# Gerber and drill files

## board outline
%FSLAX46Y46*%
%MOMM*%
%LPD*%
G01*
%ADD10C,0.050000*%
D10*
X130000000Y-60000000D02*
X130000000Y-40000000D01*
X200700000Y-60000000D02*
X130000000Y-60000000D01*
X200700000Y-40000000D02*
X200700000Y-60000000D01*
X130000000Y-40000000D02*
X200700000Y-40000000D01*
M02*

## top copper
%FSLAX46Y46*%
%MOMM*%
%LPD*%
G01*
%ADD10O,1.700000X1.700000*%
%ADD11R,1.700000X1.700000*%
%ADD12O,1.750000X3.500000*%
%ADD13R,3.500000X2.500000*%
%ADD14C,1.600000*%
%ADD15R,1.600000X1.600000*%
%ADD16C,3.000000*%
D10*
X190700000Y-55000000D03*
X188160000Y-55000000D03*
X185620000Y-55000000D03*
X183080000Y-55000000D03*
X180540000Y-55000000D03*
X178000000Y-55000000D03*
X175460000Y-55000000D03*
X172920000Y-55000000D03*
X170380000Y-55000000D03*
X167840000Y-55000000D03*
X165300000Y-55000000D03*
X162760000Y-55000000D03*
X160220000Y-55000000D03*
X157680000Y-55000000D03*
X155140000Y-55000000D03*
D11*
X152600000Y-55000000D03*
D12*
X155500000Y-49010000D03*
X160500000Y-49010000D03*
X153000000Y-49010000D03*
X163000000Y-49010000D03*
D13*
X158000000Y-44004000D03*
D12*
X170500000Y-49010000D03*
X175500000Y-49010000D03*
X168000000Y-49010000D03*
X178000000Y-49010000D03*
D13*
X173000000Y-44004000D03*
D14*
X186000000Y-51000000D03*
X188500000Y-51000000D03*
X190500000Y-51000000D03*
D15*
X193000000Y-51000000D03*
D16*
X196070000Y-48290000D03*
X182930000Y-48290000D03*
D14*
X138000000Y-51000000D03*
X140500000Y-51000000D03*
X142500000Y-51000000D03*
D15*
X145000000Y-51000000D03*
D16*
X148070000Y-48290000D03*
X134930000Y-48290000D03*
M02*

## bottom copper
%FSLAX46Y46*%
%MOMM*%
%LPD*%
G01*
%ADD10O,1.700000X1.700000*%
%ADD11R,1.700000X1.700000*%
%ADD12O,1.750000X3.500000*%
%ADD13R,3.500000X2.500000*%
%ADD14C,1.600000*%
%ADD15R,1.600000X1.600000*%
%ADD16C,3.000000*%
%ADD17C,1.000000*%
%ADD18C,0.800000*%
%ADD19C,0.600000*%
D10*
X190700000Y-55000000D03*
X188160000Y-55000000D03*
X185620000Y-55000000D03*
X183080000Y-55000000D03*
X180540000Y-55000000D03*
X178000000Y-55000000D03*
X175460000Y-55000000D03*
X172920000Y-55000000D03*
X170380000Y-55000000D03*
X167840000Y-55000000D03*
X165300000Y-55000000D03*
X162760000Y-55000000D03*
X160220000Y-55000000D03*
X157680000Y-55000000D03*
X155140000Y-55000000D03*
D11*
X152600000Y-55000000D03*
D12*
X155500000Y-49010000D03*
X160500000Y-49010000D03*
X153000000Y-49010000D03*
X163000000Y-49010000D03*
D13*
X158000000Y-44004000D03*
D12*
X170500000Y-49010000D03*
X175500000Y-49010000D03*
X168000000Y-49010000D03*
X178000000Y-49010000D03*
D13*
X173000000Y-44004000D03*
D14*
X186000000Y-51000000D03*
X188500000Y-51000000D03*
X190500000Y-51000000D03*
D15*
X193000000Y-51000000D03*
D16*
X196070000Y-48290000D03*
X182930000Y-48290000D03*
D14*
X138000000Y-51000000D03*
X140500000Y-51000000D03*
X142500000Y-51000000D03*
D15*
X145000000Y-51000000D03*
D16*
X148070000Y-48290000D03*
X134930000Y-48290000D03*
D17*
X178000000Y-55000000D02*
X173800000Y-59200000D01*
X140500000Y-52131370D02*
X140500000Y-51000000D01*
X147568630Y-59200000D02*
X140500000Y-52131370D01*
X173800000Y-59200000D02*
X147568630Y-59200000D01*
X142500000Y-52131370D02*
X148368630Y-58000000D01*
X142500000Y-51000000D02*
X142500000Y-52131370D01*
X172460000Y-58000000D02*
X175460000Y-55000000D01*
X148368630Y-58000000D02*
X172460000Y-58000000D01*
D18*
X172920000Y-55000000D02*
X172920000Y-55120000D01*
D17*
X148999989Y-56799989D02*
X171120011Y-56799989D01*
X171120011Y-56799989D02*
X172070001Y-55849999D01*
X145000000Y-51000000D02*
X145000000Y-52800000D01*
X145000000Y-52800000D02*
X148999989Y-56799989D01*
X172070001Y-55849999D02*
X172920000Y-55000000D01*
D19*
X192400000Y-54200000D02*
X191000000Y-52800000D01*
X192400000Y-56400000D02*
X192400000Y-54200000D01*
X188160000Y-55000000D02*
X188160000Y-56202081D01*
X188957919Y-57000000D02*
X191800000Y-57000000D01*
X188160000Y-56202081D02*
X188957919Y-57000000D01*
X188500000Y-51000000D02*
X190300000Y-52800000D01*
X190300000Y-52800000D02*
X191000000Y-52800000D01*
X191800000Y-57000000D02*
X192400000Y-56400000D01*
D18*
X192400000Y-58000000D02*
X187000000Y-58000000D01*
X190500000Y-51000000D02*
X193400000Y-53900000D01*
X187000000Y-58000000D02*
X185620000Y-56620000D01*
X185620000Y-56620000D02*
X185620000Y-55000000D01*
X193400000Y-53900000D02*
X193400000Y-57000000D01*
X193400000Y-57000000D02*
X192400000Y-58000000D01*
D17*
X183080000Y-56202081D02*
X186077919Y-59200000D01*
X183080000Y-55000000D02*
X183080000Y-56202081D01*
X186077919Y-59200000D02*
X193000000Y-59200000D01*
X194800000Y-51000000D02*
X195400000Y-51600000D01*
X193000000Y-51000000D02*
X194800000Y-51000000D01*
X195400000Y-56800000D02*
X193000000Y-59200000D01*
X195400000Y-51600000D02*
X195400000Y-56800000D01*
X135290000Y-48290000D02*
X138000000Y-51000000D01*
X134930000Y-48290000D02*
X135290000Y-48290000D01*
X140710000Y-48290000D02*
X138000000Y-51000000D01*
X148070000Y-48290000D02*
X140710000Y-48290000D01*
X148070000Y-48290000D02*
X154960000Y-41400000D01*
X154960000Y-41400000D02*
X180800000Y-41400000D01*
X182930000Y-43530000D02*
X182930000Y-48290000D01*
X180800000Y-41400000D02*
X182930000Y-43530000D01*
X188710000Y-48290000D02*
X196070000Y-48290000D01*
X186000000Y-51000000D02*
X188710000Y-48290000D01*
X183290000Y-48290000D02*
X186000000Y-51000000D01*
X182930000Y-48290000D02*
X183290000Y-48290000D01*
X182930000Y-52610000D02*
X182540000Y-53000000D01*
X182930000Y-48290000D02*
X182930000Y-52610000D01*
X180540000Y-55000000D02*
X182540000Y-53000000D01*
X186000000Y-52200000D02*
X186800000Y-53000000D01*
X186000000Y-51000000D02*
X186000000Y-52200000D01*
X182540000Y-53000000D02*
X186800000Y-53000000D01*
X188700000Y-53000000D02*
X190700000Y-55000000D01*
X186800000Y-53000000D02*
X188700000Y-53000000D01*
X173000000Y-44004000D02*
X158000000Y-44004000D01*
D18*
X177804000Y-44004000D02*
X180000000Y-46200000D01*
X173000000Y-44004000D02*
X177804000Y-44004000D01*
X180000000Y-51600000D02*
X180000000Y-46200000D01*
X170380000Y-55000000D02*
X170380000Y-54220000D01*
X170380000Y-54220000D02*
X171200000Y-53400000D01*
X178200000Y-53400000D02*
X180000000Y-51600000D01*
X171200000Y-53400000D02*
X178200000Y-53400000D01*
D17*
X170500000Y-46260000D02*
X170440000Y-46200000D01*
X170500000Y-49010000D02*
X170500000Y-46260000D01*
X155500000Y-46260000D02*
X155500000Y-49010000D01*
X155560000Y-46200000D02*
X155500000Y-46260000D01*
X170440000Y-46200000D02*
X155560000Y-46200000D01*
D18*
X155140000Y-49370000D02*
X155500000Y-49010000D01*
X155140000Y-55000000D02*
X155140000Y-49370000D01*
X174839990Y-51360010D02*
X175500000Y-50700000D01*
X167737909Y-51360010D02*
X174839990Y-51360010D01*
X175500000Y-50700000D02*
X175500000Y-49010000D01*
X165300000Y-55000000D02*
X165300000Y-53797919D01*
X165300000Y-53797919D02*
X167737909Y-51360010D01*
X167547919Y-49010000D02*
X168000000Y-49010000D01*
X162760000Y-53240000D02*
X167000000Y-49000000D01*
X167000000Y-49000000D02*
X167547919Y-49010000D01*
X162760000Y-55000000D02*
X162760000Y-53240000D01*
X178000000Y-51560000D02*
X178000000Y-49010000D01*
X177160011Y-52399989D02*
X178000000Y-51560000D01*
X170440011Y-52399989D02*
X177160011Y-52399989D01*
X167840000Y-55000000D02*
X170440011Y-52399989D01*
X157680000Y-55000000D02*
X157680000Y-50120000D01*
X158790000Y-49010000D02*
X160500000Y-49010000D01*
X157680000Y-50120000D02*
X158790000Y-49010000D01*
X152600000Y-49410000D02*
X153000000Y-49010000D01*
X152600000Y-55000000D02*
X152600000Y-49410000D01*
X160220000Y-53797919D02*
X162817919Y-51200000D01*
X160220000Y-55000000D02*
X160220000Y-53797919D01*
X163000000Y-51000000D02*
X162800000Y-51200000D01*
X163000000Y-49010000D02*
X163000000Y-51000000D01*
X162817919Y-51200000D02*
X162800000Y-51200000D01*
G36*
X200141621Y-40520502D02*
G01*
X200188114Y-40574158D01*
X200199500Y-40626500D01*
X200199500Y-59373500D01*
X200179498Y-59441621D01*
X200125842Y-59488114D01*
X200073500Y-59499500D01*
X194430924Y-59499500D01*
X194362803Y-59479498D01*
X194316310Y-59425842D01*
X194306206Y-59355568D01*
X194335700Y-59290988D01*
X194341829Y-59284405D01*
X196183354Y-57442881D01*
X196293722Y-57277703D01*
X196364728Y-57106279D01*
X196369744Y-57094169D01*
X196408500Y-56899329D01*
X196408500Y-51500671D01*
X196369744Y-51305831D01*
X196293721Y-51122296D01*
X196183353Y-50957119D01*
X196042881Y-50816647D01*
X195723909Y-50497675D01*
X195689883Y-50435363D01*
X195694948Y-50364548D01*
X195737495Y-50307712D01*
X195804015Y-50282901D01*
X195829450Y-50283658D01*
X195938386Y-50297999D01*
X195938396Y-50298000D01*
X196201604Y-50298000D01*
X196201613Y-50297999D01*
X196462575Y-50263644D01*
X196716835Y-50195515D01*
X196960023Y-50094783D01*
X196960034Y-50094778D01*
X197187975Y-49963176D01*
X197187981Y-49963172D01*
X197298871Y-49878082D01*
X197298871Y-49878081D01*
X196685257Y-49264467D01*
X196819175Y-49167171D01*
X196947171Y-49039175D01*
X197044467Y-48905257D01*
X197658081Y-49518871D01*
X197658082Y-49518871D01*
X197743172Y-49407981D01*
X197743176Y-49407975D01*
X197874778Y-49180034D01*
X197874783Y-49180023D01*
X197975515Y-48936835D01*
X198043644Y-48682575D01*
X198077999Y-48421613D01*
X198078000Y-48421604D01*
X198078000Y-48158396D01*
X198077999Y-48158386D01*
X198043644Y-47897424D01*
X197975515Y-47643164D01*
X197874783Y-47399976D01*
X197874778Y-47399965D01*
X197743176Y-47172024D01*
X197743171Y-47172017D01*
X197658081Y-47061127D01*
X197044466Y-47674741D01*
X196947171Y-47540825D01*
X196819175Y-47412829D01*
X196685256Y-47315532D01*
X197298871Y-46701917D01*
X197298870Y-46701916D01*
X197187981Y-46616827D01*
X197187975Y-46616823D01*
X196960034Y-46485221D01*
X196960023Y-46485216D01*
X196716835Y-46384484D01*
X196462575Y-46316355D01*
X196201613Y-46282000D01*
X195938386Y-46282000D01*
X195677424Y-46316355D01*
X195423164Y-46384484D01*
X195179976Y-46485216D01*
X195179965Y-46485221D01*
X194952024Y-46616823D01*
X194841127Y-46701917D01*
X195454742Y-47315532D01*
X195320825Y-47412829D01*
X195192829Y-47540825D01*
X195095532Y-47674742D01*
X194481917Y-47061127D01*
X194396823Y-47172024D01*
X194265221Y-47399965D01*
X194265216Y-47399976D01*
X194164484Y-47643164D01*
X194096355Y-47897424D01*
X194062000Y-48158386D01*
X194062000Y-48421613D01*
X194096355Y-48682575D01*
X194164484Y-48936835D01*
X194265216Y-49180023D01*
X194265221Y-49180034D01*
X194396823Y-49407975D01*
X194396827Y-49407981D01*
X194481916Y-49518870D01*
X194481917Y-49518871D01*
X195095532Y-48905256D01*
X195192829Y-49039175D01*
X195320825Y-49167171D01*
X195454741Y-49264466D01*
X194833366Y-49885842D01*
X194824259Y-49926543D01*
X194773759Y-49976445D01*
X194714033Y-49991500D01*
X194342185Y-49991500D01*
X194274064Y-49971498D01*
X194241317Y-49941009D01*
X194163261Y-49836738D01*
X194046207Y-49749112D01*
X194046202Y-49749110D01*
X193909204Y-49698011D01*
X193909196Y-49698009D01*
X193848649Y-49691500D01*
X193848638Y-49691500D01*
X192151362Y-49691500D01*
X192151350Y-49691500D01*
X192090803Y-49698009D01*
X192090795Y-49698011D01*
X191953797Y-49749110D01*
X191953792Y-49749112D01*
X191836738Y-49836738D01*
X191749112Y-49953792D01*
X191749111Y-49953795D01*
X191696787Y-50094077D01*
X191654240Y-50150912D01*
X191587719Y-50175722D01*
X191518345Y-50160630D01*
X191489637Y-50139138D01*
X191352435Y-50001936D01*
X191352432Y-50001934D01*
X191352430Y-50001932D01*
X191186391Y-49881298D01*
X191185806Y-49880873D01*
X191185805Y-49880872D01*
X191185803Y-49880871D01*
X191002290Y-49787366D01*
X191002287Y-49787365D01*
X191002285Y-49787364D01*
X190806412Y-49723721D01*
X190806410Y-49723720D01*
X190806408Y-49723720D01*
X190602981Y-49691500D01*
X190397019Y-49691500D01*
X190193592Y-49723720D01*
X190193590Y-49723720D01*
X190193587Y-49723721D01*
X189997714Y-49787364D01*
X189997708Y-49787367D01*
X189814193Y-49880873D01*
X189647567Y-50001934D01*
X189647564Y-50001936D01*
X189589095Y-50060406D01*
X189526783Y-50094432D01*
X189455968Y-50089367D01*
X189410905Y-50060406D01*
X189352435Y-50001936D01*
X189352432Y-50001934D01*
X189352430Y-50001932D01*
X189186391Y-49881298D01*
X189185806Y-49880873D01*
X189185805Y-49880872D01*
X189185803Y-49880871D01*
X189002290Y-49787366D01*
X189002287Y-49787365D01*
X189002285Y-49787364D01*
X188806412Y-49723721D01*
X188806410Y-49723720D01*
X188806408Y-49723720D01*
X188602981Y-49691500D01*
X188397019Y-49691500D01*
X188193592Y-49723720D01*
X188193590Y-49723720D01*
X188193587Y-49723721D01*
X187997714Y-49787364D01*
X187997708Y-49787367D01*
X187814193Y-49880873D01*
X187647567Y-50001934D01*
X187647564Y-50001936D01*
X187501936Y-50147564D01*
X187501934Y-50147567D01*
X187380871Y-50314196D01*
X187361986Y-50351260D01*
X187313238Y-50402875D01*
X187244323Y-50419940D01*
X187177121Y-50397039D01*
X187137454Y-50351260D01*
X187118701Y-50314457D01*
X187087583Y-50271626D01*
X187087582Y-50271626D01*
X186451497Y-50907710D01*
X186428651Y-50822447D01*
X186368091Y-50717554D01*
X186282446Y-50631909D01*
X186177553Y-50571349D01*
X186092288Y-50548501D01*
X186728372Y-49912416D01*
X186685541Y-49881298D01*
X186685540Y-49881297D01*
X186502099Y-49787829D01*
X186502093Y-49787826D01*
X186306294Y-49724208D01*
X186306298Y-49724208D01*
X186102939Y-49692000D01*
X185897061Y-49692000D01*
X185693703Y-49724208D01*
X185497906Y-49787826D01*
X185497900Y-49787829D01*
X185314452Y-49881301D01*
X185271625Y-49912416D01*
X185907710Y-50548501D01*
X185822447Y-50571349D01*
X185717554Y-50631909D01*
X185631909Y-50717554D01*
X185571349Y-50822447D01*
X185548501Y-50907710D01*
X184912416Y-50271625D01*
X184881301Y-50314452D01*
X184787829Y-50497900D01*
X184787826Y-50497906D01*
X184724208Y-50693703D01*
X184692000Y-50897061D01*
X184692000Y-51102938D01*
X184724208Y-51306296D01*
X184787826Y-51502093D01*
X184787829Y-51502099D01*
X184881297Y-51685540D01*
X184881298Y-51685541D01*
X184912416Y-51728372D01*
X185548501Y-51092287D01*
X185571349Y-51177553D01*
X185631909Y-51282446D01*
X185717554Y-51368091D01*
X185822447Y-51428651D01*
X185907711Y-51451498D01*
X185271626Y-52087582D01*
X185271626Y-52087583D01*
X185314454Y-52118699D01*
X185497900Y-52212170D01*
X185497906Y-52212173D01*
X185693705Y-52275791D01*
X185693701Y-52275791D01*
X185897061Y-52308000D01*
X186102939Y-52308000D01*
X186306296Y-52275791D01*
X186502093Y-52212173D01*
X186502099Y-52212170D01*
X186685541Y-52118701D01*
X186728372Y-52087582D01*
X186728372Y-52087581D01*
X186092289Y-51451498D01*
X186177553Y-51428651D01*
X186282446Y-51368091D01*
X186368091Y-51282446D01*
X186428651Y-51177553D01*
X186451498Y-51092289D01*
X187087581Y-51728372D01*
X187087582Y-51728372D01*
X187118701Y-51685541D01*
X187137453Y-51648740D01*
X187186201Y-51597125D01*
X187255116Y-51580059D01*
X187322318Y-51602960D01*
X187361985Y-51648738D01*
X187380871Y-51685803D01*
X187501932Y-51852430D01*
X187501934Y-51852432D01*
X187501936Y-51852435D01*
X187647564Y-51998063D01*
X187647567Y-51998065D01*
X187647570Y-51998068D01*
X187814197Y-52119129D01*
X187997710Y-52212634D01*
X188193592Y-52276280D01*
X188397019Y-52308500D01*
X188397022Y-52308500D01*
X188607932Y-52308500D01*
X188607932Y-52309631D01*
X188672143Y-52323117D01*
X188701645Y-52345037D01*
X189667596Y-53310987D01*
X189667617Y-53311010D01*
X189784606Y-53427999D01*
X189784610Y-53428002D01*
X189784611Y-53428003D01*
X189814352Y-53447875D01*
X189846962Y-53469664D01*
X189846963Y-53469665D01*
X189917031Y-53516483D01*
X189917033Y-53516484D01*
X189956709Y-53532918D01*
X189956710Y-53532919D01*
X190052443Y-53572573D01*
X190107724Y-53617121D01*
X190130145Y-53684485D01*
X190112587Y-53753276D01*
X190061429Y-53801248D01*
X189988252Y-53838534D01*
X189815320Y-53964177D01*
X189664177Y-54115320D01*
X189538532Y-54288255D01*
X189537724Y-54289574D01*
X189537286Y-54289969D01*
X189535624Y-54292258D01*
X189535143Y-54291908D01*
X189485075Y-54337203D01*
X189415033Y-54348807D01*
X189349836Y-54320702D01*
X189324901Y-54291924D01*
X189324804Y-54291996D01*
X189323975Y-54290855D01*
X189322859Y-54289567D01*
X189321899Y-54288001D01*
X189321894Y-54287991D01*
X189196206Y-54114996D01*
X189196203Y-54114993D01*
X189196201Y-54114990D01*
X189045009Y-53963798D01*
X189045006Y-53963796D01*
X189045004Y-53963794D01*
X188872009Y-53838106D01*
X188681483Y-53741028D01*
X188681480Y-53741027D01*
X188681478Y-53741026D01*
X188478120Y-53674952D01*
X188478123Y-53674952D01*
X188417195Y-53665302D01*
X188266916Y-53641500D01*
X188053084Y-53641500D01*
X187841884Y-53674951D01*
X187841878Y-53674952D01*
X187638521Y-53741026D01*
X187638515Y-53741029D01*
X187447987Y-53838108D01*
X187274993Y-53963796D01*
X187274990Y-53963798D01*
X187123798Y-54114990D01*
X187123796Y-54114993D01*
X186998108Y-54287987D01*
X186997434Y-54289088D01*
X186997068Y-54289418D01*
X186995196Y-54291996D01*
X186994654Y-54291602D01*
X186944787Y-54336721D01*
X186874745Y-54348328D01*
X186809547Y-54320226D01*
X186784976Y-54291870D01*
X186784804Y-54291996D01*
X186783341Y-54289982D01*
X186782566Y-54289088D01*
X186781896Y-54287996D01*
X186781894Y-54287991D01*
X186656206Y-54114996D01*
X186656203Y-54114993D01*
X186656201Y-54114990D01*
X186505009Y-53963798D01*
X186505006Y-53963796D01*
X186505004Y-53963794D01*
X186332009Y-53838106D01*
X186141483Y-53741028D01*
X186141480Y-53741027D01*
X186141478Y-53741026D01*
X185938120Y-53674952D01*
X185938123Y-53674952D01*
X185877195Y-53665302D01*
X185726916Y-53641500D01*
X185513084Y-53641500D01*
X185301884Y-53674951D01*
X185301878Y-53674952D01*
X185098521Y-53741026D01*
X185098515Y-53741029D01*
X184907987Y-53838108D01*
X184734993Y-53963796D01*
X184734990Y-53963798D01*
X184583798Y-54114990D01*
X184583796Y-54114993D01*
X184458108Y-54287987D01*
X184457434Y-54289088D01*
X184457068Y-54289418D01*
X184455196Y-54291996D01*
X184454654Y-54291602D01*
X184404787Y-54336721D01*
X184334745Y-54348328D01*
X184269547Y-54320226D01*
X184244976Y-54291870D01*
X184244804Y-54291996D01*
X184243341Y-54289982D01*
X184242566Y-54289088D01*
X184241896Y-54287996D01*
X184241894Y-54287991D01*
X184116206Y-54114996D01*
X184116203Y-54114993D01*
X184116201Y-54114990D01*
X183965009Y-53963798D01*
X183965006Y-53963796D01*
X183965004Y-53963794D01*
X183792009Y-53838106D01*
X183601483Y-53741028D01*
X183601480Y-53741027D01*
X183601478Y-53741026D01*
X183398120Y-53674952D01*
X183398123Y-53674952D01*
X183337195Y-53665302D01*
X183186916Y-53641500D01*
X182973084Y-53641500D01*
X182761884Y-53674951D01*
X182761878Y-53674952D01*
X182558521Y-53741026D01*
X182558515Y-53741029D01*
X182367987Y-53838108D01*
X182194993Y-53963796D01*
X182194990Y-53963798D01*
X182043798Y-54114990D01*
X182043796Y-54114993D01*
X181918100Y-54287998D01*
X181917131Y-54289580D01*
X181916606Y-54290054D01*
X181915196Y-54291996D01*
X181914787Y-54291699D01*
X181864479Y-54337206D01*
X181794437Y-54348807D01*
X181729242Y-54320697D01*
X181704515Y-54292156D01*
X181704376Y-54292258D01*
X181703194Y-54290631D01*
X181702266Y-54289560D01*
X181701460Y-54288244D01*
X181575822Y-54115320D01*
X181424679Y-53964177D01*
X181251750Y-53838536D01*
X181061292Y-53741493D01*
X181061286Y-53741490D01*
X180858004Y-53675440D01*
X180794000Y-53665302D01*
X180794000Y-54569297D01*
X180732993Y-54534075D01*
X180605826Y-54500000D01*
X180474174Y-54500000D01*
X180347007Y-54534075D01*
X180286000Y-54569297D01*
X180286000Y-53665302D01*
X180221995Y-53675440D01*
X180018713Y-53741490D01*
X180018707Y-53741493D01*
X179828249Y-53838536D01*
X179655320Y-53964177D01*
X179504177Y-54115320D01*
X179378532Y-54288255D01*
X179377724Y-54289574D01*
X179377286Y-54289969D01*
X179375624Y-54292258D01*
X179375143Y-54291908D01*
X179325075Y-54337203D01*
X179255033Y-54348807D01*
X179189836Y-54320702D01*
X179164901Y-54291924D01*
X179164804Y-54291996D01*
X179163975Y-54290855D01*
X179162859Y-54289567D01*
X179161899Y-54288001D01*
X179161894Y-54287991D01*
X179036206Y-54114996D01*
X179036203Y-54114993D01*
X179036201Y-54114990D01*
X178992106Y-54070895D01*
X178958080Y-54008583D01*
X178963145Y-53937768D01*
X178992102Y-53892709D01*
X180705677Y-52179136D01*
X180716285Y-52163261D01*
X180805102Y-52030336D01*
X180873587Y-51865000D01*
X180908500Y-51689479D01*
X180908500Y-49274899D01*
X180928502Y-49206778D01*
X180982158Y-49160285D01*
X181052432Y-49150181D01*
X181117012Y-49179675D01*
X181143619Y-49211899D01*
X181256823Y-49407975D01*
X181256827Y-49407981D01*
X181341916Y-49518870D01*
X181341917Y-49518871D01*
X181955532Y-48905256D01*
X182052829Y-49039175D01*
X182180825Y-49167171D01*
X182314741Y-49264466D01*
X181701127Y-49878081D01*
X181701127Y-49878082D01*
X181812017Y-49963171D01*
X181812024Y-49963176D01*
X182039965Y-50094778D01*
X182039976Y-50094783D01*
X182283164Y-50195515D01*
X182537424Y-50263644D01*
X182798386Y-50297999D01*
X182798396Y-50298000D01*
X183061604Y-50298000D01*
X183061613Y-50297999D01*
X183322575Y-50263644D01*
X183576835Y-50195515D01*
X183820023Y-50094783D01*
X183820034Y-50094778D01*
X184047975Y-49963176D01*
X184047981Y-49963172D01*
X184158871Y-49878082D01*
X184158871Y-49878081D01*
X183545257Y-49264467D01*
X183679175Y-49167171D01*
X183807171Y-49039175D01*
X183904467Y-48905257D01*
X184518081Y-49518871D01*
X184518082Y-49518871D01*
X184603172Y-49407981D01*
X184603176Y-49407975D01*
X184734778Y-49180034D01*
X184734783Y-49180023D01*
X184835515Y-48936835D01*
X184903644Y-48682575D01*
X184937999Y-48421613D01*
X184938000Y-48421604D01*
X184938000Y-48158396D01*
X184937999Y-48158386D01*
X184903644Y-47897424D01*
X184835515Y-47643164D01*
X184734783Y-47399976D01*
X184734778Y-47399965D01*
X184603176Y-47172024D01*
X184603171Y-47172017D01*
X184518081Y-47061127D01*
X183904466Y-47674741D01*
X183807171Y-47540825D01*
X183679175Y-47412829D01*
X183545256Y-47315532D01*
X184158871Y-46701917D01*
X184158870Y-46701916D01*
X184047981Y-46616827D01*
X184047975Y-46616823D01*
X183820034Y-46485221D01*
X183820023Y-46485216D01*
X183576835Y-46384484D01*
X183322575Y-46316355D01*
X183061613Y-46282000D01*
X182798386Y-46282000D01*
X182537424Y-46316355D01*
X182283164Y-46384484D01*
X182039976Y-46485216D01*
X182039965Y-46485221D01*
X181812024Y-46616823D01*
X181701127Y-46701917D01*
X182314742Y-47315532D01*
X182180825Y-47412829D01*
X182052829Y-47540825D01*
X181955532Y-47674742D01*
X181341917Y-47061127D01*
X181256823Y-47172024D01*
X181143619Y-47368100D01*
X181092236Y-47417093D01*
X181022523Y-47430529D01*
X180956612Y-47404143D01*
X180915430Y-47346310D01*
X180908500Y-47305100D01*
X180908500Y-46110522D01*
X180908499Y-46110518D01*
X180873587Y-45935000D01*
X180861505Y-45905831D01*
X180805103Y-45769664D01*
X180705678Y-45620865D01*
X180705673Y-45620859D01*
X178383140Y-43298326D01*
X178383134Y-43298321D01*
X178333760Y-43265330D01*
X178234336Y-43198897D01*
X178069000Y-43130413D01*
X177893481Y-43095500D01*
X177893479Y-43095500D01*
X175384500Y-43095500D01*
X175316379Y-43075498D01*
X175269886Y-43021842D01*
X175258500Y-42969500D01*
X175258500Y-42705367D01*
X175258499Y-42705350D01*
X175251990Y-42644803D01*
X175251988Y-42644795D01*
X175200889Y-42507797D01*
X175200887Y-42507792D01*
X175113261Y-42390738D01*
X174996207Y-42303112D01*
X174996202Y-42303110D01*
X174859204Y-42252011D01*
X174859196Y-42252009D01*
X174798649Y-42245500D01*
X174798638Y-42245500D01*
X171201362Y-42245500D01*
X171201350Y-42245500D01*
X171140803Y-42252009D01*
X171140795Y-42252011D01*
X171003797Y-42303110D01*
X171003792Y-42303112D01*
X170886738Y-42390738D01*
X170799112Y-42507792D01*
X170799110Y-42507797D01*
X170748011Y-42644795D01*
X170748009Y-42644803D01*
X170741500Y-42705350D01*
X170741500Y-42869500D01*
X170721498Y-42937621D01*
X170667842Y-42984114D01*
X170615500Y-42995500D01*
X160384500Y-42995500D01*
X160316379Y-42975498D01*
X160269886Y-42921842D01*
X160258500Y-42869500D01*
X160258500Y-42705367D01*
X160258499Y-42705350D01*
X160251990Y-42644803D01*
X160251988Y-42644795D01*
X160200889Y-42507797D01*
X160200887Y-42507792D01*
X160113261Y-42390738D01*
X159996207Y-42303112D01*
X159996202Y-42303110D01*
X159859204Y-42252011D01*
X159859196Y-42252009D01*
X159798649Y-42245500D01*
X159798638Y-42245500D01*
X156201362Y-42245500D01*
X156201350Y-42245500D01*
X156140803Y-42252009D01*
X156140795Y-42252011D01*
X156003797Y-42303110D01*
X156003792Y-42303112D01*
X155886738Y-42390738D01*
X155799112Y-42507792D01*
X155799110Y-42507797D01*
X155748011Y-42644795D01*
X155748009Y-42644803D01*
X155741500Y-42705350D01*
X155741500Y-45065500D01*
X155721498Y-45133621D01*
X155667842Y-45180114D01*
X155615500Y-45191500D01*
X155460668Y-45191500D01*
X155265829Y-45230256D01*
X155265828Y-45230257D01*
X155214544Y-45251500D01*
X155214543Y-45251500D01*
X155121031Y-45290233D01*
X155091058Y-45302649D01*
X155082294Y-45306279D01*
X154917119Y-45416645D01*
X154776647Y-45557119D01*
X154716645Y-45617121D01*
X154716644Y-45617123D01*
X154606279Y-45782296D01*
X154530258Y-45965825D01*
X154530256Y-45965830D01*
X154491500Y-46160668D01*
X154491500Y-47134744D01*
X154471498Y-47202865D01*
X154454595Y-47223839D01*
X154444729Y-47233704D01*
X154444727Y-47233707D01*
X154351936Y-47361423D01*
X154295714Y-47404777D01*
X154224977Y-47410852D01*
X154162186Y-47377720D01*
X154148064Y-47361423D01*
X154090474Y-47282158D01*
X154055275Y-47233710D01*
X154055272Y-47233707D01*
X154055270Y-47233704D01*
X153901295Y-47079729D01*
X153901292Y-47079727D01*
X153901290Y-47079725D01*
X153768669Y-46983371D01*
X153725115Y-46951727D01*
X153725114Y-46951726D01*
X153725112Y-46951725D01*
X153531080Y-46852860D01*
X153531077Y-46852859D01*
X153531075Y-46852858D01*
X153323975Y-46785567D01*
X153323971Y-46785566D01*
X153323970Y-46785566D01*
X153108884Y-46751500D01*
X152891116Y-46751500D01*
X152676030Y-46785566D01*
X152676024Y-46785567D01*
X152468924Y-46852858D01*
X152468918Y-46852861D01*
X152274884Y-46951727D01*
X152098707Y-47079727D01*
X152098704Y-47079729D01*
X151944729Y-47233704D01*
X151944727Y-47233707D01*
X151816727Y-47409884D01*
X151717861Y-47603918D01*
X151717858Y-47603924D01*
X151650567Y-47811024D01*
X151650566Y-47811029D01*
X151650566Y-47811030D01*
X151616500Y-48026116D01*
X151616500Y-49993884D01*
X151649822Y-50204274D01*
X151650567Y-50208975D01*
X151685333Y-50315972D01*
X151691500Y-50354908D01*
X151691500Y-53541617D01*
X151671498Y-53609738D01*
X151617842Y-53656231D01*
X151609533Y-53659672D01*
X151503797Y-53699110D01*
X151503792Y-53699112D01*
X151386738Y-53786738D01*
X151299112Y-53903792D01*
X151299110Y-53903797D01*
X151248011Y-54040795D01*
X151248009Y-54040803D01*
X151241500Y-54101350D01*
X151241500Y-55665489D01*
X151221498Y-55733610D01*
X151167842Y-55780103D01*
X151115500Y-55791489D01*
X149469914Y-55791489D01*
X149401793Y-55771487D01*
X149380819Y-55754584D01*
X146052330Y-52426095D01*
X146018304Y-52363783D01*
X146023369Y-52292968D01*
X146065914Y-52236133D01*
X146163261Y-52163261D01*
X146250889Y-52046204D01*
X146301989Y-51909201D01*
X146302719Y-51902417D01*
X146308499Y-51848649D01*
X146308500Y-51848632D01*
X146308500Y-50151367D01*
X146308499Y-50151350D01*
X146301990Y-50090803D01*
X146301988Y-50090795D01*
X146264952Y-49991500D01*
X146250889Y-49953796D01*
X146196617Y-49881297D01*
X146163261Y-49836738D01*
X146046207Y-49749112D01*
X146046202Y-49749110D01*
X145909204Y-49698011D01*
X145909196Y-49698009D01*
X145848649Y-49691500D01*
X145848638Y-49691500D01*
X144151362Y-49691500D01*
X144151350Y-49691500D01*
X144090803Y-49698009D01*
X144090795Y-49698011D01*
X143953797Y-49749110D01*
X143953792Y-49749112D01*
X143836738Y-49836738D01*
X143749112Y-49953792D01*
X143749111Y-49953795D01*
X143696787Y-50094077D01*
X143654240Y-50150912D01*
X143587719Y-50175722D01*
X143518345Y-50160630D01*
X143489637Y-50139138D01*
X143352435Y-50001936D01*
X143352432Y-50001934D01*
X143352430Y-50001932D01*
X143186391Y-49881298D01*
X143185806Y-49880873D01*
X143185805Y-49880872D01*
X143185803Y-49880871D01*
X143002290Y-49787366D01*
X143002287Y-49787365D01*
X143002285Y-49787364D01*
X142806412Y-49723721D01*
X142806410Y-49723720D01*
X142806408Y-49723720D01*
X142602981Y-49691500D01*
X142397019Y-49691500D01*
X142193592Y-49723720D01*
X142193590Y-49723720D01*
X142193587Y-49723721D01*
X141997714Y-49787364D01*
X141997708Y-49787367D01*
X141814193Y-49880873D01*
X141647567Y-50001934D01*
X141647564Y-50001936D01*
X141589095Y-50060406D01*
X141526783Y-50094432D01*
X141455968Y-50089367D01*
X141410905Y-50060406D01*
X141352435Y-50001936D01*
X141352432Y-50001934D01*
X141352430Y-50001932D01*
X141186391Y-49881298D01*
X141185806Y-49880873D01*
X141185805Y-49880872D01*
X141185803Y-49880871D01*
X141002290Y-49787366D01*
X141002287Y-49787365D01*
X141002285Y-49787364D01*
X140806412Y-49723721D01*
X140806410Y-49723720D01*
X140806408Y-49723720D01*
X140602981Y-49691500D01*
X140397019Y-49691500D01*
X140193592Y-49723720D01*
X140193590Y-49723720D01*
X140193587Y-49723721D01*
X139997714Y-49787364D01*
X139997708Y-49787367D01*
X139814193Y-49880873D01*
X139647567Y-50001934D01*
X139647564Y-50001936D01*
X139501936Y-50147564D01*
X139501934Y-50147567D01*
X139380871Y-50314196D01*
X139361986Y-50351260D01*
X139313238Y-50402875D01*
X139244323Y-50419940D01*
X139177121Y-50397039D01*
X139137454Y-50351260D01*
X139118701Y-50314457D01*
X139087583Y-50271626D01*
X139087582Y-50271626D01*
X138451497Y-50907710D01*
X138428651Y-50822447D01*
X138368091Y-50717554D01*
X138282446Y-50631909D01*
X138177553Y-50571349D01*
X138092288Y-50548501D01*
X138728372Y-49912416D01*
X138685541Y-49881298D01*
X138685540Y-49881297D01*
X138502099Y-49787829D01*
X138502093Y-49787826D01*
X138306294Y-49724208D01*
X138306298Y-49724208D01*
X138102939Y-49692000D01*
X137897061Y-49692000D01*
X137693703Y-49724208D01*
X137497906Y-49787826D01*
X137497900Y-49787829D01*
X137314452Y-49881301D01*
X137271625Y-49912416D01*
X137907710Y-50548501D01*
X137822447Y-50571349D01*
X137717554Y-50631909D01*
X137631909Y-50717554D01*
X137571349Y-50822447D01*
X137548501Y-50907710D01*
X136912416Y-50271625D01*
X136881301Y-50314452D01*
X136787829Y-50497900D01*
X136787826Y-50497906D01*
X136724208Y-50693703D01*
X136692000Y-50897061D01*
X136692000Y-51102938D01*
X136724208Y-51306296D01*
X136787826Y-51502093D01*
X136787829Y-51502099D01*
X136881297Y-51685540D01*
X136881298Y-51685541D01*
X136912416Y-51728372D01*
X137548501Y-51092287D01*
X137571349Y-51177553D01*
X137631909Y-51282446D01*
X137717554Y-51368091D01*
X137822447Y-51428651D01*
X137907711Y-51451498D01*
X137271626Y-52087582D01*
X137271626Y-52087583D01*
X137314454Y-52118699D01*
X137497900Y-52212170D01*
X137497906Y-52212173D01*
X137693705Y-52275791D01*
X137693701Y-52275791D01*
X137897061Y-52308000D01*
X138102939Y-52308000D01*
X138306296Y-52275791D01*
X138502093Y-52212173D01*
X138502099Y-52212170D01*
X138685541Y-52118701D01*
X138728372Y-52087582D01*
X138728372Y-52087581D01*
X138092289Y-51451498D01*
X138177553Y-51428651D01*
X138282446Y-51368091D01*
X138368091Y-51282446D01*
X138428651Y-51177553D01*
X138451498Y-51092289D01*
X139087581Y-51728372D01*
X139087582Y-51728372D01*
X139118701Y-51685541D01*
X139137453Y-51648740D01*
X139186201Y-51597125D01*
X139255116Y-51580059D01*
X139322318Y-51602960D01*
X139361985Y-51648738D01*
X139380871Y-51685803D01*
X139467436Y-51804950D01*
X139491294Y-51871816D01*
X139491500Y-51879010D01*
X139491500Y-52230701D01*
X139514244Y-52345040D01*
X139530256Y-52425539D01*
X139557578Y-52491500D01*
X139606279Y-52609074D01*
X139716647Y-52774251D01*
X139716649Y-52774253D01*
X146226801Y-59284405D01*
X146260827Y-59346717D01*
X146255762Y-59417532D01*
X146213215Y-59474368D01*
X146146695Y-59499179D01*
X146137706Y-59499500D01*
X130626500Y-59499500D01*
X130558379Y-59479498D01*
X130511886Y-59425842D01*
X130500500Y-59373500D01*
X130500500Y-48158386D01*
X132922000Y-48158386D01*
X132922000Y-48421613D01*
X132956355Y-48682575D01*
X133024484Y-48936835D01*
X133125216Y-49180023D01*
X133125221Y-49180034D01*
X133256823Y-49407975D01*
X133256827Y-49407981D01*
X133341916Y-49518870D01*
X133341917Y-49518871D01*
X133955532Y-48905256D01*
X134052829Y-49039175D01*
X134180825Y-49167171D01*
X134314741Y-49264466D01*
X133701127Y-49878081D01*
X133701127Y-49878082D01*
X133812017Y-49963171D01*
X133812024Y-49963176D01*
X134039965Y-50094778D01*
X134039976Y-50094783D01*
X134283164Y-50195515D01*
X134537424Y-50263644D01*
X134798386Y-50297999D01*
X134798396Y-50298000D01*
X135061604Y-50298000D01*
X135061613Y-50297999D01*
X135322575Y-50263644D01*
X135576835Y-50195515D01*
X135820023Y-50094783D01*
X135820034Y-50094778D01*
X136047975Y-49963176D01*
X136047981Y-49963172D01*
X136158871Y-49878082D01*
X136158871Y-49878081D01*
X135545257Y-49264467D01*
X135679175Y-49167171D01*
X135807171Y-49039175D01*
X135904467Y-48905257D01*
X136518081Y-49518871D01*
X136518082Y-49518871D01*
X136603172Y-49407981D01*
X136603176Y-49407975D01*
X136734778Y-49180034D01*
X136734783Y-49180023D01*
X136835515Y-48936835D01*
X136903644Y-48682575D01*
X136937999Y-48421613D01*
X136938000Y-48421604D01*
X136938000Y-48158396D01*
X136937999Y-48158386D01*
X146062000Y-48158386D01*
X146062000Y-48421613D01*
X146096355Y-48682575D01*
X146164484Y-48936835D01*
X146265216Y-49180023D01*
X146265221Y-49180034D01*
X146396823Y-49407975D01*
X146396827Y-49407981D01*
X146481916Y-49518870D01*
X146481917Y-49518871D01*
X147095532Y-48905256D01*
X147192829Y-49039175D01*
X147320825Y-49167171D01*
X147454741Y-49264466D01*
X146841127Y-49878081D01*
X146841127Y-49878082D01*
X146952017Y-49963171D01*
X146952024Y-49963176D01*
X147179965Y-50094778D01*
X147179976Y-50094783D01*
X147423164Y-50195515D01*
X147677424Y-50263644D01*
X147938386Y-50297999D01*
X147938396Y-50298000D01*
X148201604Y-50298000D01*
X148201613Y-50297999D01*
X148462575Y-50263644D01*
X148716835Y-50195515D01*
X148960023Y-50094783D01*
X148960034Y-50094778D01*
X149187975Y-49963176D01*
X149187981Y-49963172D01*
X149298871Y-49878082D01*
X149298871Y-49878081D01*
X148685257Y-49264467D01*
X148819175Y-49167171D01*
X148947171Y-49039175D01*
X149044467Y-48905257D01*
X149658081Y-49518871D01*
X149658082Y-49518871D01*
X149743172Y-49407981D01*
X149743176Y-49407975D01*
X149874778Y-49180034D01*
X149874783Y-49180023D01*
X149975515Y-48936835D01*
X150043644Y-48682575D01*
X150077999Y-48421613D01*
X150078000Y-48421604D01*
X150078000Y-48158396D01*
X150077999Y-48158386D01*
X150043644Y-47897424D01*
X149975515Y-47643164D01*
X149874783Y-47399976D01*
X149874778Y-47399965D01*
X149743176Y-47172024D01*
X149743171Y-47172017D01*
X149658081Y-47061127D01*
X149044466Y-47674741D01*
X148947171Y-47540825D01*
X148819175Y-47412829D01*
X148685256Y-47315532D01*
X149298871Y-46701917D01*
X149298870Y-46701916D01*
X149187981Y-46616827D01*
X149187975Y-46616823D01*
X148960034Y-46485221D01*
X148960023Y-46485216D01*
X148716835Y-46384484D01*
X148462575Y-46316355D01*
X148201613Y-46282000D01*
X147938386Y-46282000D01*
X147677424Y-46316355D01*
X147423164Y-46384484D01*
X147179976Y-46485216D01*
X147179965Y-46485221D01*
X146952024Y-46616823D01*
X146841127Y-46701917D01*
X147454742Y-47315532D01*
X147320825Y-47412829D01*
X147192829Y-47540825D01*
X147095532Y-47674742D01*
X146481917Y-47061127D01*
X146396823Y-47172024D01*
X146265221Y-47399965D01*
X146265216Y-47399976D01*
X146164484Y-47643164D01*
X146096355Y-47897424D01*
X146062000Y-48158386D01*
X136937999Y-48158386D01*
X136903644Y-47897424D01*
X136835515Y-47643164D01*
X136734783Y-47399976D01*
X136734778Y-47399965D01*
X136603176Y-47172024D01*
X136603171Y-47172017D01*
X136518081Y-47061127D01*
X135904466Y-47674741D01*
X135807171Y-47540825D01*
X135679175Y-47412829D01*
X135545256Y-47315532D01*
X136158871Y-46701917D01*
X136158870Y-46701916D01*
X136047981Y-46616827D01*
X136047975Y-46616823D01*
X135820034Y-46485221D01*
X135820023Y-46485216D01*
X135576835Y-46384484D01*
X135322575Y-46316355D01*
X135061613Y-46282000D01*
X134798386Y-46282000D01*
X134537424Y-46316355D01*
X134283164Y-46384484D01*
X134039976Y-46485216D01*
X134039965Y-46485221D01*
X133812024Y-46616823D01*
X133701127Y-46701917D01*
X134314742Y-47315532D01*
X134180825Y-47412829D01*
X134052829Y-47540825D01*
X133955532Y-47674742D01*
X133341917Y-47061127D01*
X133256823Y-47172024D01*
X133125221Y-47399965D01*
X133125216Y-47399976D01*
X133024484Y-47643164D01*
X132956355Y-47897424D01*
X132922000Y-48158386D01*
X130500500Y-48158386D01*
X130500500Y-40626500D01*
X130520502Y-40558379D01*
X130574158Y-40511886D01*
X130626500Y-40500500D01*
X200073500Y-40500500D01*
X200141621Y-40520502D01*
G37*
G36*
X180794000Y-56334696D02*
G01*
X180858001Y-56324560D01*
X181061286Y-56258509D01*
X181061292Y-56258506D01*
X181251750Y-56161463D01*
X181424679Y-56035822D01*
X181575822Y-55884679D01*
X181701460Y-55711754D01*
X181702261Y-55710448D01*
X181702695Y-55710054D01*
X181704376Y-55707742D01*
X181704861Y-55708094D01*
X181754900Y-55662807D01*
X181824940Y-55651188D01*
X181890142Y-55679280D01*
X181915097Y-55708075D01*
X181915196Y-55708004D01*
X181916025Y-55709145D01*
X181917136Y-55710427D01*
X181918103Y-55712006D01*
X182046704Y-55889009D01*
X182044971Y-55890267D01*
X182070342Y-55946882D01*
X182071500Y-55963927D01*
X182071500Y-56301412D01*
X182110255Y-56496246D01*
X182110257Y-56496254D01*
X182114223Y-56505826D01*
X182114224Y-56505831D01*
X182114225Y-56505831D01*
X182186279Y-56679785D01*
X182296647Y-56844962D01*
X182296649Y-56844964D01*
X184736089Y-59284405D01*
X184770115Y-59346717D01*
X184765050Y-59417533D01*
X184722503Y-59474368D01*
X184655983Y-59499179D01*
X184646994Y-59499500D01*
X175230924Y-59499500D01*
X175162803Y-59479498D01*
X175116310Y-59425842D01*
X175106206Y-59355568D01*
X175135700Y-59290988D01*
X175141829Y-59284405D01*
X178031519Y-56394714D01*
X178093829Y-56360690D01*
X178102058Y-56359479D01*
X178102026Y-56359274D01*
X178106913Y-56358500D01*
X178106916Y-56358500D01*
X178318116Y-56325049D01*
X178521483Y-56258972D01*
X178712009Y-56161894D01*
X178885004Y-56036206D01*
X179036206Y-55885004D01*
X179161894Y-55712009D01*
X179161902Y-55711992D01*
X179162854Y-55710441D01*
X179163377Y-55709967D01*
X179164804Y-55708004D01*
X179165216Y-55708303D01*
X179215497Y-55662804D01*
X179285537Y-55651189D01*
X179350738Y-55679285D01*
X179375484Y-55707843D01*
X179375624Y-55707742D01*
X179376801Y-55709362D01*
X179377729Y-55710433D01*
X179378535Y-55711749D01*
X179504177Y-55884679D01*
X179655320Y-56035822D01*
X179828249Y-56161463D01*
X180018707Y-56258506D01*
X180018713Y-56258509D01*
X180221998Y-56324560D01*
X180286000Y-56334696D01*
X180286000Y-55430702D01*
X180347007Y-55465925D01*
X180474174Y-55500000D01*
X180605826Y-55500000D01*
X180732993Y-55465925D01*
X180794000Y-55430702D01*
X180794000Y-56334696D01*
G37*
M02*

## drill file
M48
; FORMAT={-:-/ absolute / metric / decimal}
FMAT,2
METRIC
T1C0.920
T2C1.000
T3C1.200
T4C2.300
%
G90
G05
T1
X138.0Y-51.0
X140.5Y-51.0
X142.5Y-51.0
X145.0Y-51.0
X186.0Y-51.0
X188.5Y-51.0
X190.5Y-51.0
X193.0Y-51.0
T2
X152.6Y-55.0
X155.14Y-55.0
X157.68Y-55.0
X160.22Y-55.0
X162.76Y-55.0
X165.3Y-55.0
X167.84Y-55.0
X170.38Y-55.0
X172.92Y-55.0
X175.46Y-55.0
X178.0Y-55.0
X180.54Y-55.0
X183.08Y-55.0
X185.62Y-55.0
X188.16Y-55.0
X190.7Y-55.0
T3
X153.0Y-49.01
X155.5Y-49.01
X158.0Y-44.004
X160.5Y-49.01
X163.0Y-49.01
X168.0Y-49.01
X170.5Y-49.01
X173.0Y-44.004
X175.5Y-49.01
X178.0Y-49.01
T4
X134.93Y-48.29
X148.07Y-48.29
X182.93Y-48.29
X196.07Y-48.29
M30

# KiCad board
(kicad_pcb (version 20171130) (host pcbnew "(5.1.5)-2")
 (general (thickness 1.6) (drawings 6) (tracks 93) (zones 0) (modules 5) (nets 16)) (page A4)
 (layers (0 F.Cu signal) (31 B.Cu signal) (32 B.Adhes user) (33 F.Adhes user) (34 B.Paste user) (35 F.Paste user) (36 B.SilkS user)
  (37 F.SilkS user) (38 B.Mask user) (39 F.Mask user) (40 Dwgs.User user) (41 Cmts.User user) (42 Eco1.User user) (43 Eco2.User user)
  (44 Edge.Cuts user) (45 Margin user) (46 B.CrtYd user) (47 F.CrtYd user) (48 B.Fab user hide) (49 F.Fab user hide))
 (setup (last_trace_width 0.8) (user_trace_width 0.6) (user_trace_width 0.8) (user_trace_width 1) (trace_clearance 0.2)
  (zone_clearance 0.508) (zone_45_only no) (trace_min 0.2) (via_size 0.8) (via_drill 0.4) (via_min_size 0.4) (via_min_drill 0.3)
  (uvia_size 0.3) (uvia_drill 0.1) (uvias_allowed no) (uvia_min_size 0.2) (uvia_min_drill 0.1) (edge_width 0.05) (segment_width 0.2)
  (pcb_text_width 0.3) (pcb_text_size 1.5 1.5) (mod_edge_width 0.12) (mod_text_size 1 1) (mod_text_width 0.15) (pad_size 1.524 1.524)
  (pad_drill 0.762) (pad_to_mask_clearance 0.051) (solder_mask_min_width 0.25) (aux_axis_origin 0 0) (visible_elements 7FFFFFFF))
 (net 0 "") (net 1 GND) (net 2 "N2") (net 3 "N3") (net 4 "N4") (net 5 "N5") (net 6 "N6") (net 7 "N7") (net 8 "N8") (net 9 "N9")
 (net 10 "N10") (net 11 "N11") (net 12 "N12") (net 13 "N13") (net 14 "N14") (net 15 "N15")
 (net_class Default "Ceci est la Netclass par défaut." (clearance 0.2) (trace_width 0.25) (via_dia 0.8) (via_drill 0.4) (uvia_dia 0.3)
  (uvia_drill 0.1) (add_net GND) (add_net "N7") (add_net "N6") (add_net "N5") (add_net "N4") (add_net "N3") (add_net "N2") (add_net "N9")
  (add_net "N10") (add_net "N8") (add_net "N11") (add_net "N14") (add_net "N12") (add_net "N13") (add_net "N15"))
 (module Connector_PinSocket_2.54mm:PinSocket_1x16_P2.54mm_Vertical (layer F.Cu) (at 152.6 55 90)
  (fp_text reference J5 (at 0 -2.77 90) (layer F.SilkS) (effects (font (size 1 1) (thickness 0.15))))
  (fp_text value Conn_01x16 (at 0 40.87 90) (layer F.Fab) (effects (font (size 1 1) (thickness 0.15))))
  (pad 16 thru_hole oval (at 0 38.1 90) (size 1.7 1.7) (drill 1) (layers *.Cu *.Mask) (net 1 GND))
  (pad 15 thru_hole oval (at 0 35.56 90) (size 1.7 1.7) (drill 1) (layers *.Cu *.Mask) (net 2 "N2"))
  (pad 14 thru_hole oval (at 0 33.02 90) (size 1.7 1.7) (drill 1) (layers *.Cu *.Mask) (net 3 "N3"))
  (pad 13 thru_hole oval (at 0 30.48 90) (size 1.7 1.7) (drill 1) (layers *.Cu *.Mask) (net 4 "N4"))
  (pad 12 thru_hole oval (at 0 27.94 90) (size 1.7 1.7) (drill 1) (layers *.Cu *.Mask) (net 1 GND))
  (pad 11 thru_hole oval (at 0 25.4 90) (size 1.7 1.7) (drill 1) (layers *.Cu *.Mask) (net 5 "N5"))
  (pad 10 thru_hole oval (at 0 22.86 90) (size 1.7 1.7) (drill 1) (layers *.Cu *.Mask) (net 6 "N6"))
  (pad 9 thru_hole oval (at 0 20.32 90) (size 1.7 1.7) (drill 1) (layers *.Cu *.Mask) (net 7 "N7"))
  (pad 8 thru_hole oval (at 0 17.78 90) (size 1.7 1.7) (drill 1) (layers *.Cu *.Mask) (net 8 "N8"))
  (pad 7 thru_hole oval (at 0 15.24 90) (size 1.7 1.7) (drill 1) (layers *.Cu *.Mask) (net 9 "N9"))
  (pad 6 thru_hole oval (at 0 12.7 90) (size 1.7 1.7) (drill 1) (layers *.Cu *.Mask) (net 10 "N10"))
  (pad 5 thru_hole oval (at 0 10.16 90) (size 1.7 1.7) (drill 1) (layers *.Cu *.Mask) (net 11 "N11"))
  (pad 4 thru_hole oval (at 0 7.62 90) (size 1.7 1.7) (drill 1) (layers *.Cu *.Mask) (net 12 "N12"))
  (pad 3 thru_hole oval (at 0 5.08 90) (size 1.7 1.7) (drill 1) (layers *.Cu *.Mask) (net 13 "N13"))
  (pad 2 thru_hole oval (at 0 2.54 90) (size 1.7 1.7) (drill 1) (layers *.Cu *.Mask) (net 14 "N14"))
  (pad 1 thru_hole rect (at 0 0 90) (size 1.7 1.7) (drill 1) (layers *.Cu *.Mask) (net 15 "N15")))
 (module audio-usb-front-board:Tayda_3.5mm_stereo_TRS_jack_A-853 (layer F.Cu) (at 158 45.6)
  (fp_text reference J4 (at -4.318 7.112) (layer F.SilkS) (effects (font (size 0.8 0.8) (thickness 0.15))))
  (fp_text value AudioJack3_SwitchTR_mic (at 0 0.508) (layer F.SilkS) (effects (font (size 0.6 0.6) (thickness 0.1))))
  (pad TN thru_hole oval (at -2.5 3.41) (size 1.75 3.5) (drill 1.2) (layers *.Cu *.Mask F.SilkS) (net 14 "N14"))
  (pad RN thru_hole oval (at 2.5 3.41) (size 1.75 3.5) (drill 1.2) (layers *.Cu *.Mask F.SilkS) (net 13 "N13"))
  (pad T thru_hole oval (at -5 3.41) (size 1.75 3.5) (drill 1.2) (layers *.Cu *.Mask F.SilkS) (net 15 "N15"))
  (pad R thru_hole oval (at 5 3.41) (size 1.75 3.5) (drill 1.2) (layers *.Cu *.Mask F.SilkS) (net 12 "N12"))
  (pad S thru_hole rect (at 0 -1.596) (size 3.5 2.5) (drill 1.2) (layers *.Cu *.Mask F.SilkS) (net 8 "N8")))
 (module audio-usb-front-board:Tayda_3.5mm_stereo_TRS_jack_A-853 (layer F.Cu) (at 173 45.6)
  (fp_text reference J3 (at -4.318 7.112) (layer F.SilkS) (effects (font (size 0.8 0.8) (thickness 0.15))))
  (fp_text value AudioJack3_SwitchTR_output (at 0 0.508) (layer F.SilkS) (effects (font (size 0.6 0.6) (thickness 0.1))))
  (pad TN thru_hole oval (at -2.5 3.41) (size 1.75 3.5) (drill 1.2) (layers *.Cu *.Mask F.SilkS) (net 14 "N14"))
  (pad RN thru_hole oval (at 2.5 3.41) (size 1.75 3.5) (drill 1.2) (layers *.Cu *.Mask F.SilkS) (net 10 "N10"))
  (pad T thru_hole oval (at -5 3.41) (size 1.75 3.5) (drill 1.2) (layers *.Cu *.Mask F.SilkS) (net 11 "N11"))
  (pad R thru_hole oval (at 5 3.41) (size 1.75 3.5) (drill 1.2) (layers *.Cu *.Mask F.SilkS) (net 9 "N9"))
  (pad S thru_hole rect (at 0 -1.596) (size 3.5 2.5) (drill 1.2) (layers *.Cu *.Mask F.SilkS) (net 8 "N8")))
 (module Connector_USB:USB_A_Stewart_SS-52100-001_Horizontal (layer F.Cu) (at 193 51 180)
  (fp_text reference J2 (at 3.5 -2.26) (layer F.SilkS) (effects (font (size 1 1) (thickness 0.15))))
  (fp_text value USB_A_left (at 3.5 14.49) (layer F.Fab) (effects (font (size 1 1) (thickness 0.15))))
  (pad 4 thru_hole circle (at 7 0 180) (size 1.6 1.6) (drill 0.92) (layers *.Cu *.Mask) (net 1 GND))
  (pad 3 thru_hole circle (at 4.5 0 180) (size 1.6 1.6) (drill 0.92) (layers *.Cu *.Mask) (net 2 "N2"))
  (pad 2 thru_hole circle (at 2.5 0 180) (size 1.6 1.6) (drill 0.92) (layers *.Cu *.Mask) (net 3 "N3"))
  (pad 1 thru_hole rect (at 0 0 180) (size 1.6 1.6) (drill 0.92) (layers *.Cu *.Mask) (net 4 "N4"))
  (pad 5 thru_hole circle (at -3.07 2.71 180) (size 3 3) (drill 2.3) (layers *.Cu *.Mask) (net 1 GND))
  (pad 5 thru_hole circle (at 10.07 2.71 180) (size 3 3) (drill 2.3) (layers *.Cu *.Mask) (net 1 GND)))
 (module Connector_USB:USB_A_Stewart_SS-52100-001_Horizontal (layer F.Cu) (at 145 51 180)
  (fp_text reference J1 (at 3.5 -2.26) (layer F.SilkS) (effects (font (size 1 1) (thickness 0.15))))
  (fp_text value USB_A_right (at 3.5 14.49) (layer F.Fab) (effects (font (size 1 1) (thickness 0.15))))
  (pad 4 thru_hole circle (at 7 0 180) (size 1.6 1.6) (drill 0.92) (layers *.Cu *.Mask) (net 1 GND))
  (pad 3 thru_hole circle (at 4.5 0 180) (size 1.6 1.6) (drill 0.92) (layers *.Cu *.Mask) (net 5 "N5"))
  (pad 2 thru_hole circle (at 2.5 0 180) (size 1.6 1.6) (drill 0.92) (layers *.Cu *.Mask) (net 6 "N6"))
  (pad 1 thru_hole rect (at 0 0 180) (size 1.6 1.6) (drill 0.92) (layers *.Cu *.Mask) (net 7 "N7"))
  (pad 5 thru_hole circle (at -3.07 2.71 180) (size 3 3) (drill 2.3) (layers *.Cu *.Mask) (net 1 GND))
  (pad 5 thru_hole circle (at 10.07 2.71 180) (size 3 3) (drill 2.3) (layers *.Cu *.Mask) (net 1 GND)))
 (gr_line (start 130 60) (end 130 40) (layer Edge.Cuts) (width 0.05))
 (gr_line (start 200.7 60) (end 130 60) (layer Edge.Cuts) (width 0.05))
 (gr_line (start 200.7 40) (end 200.7 60) (layer Edge.Cuts) (width 0.05))
 (gr_line (start 130 40) (end 200.7 40) (layer Edge.Cuts) (width 0.05))
 (segment (start 178 55) (end 173.8 59.2) (width 1) (layer B.Cu) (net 5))
 (segment (start 140.5 52.13137) (end 140.5 51) (width 1) (layer B.Cu) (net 5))
 (segment (start 147.56863 59.2) (end 140.5 52.13137) (width 1) (layer B.Cu) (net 5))
 (segment (start 173.8 59.2) (end 147.56863 59.2) (width 1) (layer B.Cu) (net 5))
 (segment (start 142.5 52.13137) (end 148.36863 58) (width 1) (layer B.Cu) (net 6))
 (segment (start 142.5 51) (end 142.5 52.13137) (width 1) (layer B.Cu) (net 6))
 (segment (start 172.46 58) (end 175.46 55) (width 1) (layer B.Cu) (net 6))
 (segment (start 148.36863 58) (end 172.46 58) (width 1) (layer B.Cu) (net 6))
 (segment (start 172.92 55) (end 172.92 55.12) (width 0.8) (layer B.Cu) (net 7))
 (segment (start 148.999989 56.799989) (end 171.120011 56.799989) (width 1) (layer B.Cu) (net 7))
 (segment (start 171.120011 56.799989) (end 172.070001 55.849999) (width 1) (layer B.Cu) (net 7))
 (segment (start 145 51) (end 145 52.8) (width 1) (layer B.Cu) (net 7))
 (segment (start 145 52.8) (end 148.999989 56.799989) (width 1) (layer B.Cu) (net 7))
 (segment (start 172.070001 55.849999) (end 172.92 55) (width 1) (layer B.Cu) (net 7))
 (segment (start 192.4 54.2) (end 191 52.8) (width 0.6) (layer B.Cu) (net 2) (status 1000000))
 (segment (start 192.4 56.4) (end 192.4 54.2) (width 0.6) (layer B.Cu) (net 2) (status 1000000))
 (segment (start 188.16 55) (end 188.16 56.202081) (width 0.6) (layer B.Cu) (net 2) (status 1000000))
 (segment (start 188.957919 57) (end 191.8 57) (width 0.6) (layer B.Cu) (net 2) (status 1000000))
 (segment (start 188.16 56.202081) (end 188.957919 57) (width 0.6) (layer B.Cu) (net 2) (status 1000000))
 (segment (start 188.5 51) (end 190.3 52.8) (width 0.6) (layer B.Cu) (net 2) (status 1000000))
 (segment (start 190.3 52.8) (end 191 52.8) (width 0.6) (layer B.Cu) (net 2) (status 1000000))
 (segment (start 191.8 57) (end 192.4 56.4) (width 0.6) (layer B.Cu) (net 2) (status 1000000))
 (segment (start 192.4 58) (end 187 58) (width 0.8) (layer B.Cu) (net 3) (status 1000000))
 (segment (start 190.5 51) (end 193.4 53.9) (width 0.8) (layer B.Cu) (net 3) (status 1000000))
 (segment (start 187 58) (end 185.62 56.62) (width 0.8) (layer B.Cu) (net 3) (status 1000000))
 (segment (start 185.62 56.62) (end 185.62 55) (width 0.8) (layer B.Cu) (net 3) (status 1000000))
 (segment (start 193.4 53.9) (end 193.4 57) (width 0.8) (layer B.Cu) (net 3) (status 1000000))
 (segment (start 193.4 57) (end 192.4 58) (width 0.8) (layer B.Cu) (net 3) (status 1000000))
 (segment (start 183.08 56.202081) (end 186.077919 59.2) (width 1) (layer B.Cu) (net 4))
 (segment (start 183.08 55) (end 183.08 56.202081) (width 1) (layer B.Cu) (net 4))
 (segment (start 186.077919 59.2) (end 193 59.2) (width 1) (layer B.Cu) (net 4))
 (segment (start 194.8 51) (end 195.4 51.6) (width 1) (layer B.Cu) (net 4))
 (segment (start 193 51) (end 194.8 51) (width 1) (layer B.Cu) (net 4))
 (segment (start 195.4 56.8) (end 193 59.2) (width 1) (layer B.Cu) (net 4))
 (segment (start 195.4 51.6) (end 195.4 56.8) (width 1) (layer B.Cu) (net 4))
 (segment (start 135.29 48.29) (end 138 51) (width 1) (layer B.Cu) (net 1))
 (segment (start 134.93 48.29) (end 135.29 48.29) (width 1) (layer B.Cu) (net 1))
 (segment (start 140.71 48.29) (end 138 51) (width 1) (layer B.Cu) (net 1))
 (segment (start 148.07 48.29) (end 140.71 48.29) (width 1) (layer B.Cu) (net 1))
 (segment (start 148.07 48.29) (end 154.96 41.4) (width 1) (layer B.Cu) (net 1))
 (segment (start 154.96 41.4) (end 180.8 41.4) (width 1) (layer B.Cu) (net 1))
 (segment (start 182.93 43.53) (end 182.93 48.29) (width 1) (layer B.Cu) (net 1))
 (segment (start 180.8 41.4) (end 182.93 43.53) (width 1) (layer B.Cu) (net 1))
 (segment (start 188.71 48.29) (end 196.07 48.29) (width 1) (layer B.Cu) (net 1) (status 1000000))
 (segment (start 186 51) (end 188.71 48.29) (width 1) (layer B.Cu) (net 1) (status 1000000))
 (segment (start 183.29 48.29) (end 186 51) (width 1) (layer B.Cu) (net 1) (status 1000000))
 (segment (start 182.93 48.29) (end 183.29 48.29) (width 1) (layer B.Cu) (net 1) (status 1000000))
 (segment (start 182.93 52.61) (end 182.54 53) (width 1) (layer B.Cu) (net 1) (status 1000000))
 (segment (start 182.93 48.29) (end 182.93 52.61) (width 1) (layer B.Cu) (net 1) (status 1000000))
 (segment (start 180.54 55) (end 182.54 53) (width 1) (layer B.Cu) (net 1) (status 1000000))
 (segment (start 186 52.2) (end 186.8 53) (width 1) (layer B.Cu) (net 1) (status 1000000))
 (segment (start 186 51) (end 186 52.2) (width 1) (layer B.Cu) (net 1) (status 1000000))
 (segment (start 182.54 53) (end 186.8 53) (width 1) (layer B.Cu) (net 1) (status 1000000))
 (segment (start 188.7 53) (end 190.7 55) (width 1) (layer B.Cu) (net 1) (status 1000000))
 (segment (start 186.8 53) (end 188.7 53) (width 1) (layer B.Cu) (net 1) (status 1000000))
 (segment (start 173 44.004) (end 158 44.004) (width 1) (layer B.Cu) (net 8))
 (segment (start 177.804 44.004) (end 180 46.2) (width 0.8) (layer B.Cu) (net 8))
 (segment (start 173 44.004) (end 177.804 44.004) (width 0.8) (layer B.Cu) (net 8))
 (segment (start 180 51.6) (end 180 46.2) (width 0.8) (layer B.Cu) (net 8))
 (segment (start 170.38 55) (end 170.38 54.22) (width 0.8) (layer B.Cu) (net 8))
 (segment (start 170.38 54.22) (end 171.2 53.4) (width 0.8) (layer B.Cu) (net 8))
 (segment (start 178.2 53.4) (end 180 51.6) (width 0.8) (layer B.Cu) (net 8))
 (segment (start 171.2 53.4) (end 178.2 53.4) (width 0.8) (layer B.Cu) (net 8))
 (segment (start 170.5 46.26) (end 170.44 46.2) (width 1) (layer B.Cu) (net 14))
 (segment (start 170.5 49.01) (end 170.5 46.26) (width 1) (layer B.Cu) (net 14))
 (segment (start 155.5 46.26) (end 155.5 49.01) (width 1) (layer B.Cu) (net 14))
 (segment (start 155.56 46.2) (end 155.5 46.26) (width 1) (layer B.Cu) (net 14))
 (segment (start 170.44 46.2) (end 155.56 46.2) (width 1) (layer B.Cu) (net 14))
 (segment (start 155.14 49.37) (end 155.5 49.01) (width 0.8) (layer B.Cu) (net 14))
 (segment (start 155.14 55) (end 155.14 49.37) (width 0.8) (layer B.Cu) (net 14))
 (segment (start 174.83999 51.36001) (end 175.5 50.7) (width 0.8) (layer B.Cu) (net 10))
 (segment (start 167.737909 51.36001) (end 174.83999 51.36001) (width 0.8) (layer B.Cu) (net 10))
 (segment (start 175.5 50.7) (end 175.5 49.01) (width 0.8) (layer B.Cu) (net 10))
 (segment (start 165.3 55) (end 165.3 53.797919) (width 0.8) (layer B.Cu) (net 10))
 (segment (start 165.3 53.797919) (end 167.737909 51.36001) (width 0.8) (layer B.Cu) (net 10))
 (segment (start 167.547919 49.01) (end 168 49.01) (width 0.8) (layer B.Cu) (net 11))
 (segment (start 162.76 53.24) (end 167 49) (width 0.8) (layer B.Cu) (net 11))
 (segment (start 167 49) (end 167.547919 49.01) (width 0.8) (layer B.Cu) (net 11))
 (segment (start 162.76 55) (end 162.76 53.24) (width 0.8) (layer B.Cu) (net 11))
 (segment (start 178 51.56) (end 178 49.01) (width 0.8) (layer B.Cu) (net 9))
 (segment (start 177.160011 52.399989) (end 178 51.56) (width 0.8) (layer B.Cu) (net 9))
 (segment (start 170.440011 52.399989) (end 177.160011 52.399989) (width 0.8) (layer B.Cu) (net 9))
 (segment (start 167.84 55) (end 170.440011 52.399989) (width 0.8) (layer B.Cu) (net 9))
 (segment (start 157.68 55) (end 157.68 50.12) (width 0.8) (layer B.Cu) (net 13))
 (segment (start 158.79 49.01) (end 160.5 49.01) (width 0.8) (layer B.Cu) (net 13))
 (segment (start 157.68 50.12) (end 158.79 49.01) (width 0.8) (layer B.Cu) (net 13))
 (segment (start 152.6 49.41) (end 153 49.01) (width 0.8) (layer B.Cu) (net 15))
 (segment (start 152.6 55) (end 152.6 49.41) (width 0.8) (layer B.Cu) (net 15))
 (segment (start 160.22 53.797919) (end 162.817919 51.2) (width 0.8) (layer B.Cu) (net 12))
 (segment (start 160.22 55) (end 160.22 53.797919) (width 0.8) (layer B.Cu) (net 12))
 (segment (start 163 51) (end 162.8 51.2) (width 0.8) (layer B.Cu) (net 12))
 (segment (start 163 49.01) (end 163 51) (width 0.8) (layer B.Cu) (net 12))
 (segment (start 162.817919 51.2) (end 162.8 51.2) (width 0.8) (layer B.Cu) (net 12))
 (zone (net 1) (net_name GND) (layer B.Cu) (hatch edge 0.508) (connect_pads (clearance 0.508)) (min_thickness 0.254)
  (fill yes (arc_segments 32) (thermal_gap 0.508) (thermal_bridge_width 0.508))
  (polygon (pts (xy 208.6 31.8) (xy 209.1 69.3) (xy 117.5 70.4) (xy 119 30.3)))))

